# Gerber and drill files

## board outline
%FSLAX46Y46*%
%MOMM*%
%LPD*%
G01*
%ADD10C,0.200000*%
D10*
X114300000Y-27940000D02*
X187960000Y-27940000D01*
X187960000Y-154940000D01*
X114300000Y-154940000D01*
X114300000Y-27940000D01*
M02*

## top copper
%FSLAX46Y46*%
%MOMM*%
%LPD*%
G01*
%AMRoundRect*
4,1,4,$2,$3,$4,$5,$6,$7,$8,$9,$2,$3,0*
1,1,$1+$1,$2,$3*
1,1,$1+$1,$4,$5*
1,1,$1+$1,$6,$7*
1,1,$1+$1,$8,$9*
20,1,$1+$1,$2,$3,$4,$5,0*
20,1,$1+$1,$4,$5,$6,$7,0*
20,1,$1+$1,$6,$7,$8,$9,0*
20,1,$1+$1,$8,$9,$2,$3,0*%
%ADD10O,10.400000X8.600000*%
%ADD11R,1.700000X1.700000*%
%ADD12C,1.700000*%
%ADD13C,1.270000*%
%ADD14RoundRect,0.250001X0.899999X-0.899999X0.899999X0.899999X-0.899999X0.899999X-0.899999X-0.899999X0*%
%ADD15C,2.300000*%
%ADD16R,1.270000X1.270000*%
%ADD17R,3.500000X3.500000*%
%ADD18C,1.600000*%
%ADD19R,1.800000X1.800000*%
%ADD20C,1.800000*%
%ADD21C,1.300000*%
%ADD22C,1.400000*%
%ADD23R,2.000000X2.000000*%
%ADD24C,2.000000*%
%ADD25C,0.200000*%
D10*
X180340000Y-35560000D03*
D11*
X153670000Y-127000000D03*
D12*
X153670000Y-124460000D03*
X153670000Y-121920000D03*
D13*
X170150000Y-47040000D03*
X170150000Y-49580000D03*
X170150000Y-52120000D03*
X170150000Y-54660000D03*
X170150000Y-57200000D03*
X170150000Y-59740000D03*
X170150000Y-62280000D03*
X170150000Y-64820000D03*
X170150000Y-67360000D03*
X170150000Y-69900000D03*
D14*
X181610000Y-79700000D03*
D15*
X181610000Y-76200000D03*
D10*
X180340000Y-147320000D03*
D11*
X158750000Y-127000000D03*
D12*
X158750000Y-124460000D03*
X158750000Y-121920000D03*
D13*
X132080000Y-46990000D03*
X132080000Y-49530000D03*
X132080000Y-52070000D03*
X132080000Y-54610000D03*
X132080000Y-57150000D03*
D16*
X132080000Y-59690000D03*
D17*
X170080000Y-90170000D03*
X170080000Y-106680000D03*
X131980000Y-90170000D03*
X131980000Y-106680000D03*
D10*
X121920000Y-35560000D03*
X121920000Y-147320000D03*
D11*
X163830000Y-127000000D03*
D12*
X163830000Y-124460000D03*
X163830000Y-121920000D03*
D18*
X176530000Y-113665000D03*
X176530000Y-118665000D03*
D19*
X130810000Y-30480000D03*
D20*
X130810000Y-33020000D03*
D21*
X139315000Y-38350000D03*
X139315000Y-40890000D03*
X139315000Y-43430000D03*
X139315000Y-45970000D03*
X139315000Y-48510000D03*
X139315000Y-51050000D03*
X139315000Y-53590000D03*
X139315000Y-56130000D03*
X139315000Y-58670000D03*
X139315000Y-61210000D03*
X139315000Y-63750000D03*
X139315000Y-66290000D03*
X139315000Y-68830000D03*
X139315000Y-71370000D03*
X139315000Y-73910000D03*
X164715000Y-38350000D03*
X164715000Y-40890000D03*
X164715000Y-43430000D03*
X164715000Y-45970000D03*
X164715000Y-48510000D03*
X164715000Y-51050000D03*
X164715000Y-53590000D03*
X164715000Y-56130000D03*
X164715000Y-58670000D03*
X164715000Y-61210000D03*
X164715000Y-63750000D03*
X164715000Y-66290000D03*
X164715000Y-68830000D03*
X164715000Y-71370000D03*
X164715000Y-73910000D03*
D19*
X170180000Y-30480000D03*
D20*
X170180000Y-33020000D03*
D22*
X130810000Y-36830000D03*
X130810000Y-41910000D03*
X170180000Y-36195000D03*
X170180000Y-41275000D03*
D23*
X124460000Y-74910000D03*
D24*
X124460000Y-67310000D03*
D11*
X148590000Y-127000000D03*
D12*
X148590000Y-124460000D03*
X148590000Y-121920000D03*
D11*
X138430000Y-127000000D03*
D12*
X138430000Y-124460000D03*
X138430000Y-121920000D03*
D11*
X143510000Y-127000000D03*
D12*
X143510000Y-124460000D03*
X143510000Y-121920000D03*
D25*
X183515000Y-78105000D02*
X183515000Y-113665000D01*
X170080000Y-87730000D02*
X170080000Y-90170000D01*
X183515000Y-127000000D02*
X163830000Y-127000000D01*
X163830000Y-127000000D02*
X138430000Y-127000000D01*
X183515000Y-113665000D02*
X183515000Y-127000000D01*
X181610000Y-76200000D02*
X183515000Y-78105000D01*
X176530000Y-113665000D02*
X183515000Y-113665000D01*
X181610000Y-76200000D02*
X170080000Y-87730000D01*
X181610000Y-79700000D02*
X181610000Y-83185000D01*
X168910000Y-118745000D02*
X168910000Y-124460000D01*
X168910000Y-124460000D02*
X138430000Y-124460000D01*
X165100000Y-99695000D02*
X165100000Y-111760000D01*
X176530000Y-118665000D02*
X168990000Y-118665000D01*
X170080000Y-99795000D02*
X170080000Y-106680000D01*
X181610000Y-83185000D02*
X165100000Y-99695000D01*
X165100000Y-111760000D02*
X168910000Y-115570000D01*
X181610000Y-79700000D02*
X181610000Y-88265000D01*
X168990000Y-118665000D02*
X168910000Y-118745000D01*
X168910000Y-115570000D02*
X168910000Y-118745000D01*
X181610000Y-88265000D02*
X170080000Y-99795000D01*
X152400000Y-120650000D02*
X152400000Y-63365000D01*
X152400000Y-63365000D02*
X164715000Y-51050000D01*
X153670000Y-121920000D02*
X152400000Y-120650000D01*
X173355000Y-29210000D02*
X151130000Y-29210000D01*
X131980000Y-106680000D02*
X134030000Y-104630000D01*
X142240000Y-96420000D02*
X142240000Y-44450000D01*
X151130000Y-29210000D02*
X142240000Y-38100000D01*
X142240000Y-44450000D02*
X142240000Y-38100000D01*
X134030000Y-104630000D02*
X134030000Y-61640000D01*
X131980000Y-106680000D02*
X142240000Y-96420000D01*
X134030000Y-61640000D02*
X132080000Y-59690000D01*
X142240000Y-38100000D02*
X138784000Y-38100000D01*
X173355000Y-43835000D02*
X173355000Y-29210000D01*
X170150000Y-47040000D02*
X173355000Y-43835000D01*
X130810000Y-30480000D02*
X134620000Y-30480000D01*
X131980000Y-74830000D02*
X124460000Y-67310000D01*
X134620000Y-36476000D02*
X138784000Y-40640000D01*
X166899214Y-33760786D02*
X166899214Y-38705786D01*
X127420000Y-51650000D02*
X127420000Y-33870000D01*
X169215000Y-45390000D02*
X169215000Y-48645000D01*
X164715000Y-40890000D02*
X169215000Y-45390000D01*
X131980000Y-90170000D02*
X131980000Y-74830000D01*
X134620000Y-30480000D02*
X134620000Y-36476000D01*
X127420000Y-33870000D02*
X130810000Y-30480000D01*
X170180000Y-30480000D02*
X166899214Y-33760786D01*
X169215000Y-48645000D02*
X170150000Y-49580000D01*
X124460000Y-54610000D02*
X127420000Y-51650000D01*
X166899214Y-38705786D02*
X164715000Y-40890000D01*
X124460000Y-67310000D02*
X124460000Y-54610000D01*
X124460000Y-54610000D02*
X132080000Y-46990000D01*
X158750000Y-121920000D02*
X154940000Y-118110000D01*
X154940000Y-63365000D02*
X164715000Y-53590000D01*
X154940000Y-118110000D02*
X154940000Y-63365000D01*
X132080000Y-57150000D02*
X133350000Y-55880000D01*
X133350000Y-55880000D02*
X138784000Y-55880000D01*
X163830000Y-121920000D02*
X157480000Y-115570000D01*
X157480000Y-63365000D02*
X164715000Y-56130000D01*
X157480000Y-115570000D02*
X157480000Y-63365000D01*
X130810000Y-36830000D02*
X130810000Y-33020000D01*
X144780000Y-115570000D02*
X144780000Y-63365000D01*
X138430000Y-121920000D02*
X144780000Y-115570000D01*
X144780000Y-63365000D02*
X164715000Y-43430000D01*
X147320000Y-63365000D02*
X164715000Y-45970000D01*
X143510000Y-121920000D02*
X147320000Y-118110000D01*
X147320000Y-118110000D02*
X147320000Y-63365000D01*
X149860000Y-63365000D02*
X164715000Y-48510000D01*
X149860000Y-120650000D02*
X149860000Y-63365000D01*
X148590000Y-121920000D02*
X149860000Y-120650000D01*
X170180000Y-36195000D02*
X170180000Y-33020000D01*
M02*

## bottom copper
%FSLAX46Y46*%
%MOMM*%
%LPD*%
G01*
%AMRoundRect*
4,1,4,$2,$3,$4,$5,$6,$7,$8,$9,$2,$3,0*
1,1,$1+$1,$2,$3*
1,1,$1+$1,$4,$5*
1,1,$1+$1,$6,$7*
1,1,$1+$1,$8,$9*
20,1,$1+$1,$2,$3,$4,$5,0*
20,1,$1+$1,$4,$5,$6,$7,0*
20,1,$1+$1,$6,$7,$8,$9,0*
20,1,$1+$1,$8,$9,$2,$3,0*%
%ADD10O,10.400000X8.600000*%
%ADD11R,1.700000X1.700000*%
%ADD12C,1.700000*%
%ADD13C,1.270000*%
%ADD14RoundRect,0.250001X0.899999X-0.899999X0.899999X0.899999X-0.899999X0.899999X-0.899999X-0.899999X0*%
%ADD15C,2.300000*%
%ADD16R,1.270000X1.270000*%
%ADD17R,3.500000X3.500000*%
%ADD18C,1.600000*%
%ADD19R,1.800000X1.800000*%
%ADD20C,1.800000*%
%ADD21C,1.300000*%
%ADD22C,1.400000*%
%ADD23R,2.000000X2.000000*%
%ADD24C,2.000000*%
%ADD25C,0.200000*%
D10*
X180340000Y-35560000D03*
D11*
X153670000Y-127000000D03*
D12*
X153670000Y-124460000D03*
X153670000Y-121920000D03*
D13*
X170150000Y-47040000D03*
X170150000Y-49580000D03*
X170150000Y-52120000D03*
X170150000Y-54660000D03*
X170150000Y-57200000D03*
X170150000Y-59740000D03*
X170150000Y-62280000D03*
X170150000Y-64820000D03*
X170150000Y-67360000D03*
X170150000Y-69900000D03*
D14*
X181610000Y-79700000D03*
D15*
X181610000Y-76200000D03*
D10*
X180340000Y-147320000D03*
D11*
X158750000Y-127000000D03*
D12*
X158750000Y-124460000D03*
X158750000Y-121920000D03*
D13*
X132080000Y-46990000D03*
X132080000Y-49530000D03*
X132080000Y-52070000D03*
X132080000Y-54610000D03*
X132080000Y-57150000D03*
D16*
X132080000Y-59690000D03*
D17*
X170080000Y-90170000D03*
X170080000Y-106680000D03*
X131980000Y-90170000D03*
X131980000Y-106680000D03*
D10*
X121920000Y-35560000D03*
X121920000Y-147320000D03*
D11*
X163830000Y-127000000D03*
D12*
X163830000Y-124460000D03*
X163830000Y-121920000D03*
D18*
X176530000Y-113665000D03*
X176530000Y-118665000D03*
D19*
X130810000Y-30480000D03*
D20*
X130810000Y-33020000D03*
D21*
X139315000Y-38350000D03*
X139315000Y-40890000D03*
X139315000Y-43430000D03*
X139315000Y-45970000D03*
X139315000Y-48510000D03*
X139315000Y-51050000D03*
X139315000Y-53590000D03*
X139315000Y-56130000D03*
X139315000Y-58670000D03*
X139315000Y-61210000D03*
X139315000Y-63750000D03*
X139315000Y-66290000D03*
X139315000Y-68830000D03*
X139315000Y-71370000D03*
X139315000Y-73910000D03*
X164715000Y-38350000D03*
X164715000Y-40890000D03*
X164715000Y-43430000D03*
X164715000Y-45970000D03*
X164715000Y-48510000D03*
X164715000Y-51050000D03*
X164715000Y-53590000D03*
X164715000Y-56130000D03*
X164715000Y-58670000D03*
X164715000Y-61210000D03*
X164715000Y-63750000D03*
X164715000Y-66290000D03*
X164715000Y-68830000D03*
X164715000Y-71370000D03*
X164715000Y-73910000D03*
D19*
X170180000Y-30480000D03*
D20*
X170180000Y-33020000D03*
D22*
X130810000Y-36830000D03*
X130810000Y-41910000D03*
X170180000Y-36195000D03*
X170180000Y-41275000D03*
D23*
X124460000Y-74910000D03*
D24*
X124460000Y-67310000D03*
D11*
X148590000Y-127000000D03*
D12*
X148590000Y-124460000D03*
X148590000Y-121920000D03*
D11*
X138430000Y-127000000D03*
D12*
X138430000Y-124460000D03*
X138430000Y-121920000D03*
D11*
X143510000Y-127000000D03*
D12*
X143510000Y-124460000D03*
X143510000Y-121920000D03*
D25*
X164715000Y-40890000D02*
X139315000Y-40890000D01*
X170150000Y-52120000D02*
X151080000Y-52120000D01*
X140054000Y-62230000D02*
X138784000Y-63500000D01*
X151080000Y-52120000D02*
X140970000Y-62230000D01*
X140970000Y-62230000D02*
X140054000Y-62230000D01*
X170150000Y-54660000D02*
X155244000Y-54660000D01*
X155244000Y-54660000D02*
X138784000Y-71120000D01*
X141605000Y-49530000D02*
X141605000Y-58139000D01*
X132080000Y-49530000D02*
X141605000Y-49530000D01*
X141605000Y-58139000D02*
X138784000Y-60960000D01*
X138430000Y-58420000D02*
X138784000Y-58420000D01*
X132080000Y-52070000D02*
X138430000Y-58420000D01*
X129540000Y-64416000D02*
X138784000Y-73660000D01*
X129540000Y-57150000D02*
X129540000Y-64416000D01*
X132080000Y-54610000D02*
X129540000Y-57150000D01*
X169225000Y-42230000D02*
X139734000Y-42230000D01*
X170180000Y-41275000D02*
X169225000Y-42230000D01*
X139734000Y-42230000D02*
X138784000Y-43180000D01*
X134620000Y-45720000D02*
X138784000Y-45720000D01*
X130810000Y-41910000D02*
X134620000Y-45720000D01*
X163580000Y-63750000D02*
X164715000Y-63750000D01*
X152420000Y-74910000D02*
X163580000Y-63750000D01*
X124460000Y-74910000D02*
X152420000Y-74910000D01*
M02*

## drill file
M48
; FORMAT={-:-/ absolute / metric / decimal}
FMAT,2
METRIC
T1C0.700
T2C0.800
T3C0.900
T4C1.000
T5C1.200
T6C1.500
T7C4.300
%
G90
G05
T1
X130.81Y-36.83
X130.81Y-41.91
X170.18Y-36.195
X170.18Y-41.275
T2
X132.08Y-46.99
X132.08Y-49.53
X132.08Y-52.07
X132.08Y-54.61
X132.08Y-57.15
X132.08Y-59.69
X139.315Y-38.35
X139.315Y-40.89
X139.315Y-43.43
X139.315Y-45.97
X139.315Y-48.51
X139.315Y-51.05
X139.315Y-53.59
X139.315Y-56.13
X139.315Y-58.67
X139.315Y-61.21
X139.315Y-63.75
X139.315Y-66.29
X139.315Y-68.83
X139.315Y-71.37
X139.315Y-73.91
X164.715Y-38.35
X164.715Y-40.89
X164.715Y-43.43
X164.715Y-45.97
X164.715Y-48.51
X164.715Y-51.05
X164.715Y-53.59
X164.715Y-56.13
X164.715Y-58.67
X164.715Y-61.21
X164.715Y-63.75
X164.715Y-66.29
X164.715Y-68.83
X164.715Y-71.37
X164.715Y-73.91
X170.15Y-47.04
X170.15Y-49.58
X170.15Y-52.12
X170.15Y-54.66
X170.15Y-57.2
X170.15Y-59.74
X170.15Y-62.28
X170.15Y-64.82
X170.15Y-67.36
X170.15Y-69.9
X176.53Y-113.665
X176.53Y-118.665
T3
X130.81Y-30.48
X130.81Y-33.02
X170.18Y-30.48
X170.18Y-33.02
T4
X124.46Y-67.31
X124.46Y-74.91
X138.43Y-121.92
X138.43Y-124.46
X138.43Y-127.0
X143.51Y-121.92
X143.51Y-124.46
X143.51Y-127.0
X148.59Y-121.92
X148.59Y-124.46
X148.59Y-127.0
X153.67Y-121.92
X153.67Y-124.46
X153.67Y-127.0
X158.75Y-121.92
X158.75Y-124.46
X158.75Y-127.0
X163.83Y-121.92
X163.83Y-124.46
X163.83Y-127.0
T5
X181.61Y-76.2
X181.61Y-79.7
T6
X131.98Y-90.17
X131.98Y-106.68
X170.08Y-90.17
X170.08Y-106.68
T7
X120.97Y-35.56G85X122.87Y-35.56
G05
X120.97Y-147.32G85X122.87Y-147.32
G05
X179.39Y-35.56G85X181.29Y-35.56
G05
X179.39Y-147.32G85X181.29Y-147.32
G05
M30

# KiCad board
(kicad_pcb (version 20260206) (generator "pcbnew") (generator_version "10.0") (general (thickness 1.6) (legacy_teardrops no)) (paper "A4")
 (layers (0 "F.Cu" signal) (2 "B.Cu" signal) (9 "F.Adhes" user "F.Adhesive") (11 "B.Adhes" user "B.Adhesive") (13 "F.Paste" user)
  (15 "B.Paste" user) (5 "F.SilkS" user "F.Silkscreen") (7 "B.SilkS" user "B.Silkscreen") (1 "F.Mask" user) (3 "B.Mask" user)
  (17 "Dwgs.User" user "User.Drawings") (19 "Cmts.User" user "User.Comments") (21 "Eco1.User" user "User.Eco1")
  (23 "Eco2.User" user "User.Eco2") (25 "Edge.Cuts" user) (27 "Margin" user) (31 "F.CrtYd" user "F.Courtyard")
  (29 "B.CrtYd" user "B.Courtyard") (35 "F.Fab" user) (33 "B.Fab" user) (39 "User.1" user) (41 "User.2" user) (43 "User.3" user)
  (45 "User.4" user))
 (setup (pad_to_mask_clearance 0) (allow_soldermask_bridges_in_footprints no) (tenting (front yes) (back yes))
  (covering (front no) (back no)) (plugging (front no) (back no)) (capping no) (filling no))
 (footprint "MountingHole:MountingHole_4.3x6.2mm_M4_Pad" (layer "F.Cu") (at 180.34 35.56)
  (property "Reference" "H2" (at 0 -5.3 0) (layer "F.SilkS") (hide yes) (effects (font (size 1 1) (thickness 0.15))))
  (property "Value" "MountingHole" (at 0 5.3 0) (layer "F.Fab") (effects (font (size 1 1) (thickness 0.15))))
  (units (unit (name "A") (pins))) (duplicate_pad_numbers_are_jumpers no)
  (pad "1" thru_hole oval (at 0 0) (size 10.4 8.6) (drill oval 6.2 4.3) (layers "*.Cu" "*.Mask") (remove_unused_layers no)))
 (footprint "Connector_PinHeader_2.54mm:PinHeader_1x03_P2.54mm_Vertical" (layer "F.Cu") (at 153.67 127 180)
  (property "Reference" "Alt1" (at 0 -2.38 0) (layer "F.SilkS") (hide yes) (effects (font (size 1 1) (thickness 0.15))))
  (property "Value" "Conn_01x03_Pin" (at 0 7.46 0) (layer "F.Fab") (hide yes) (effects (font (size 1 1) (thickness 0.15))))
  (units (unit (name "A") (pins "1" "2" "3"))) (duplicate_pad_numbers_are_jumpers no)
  (pad "1" thru_hole rect (at 0 0 180) (size 1.7 1.7) (drill 1) (layers "*.Cu" "*.Mask") (remove_unused_layers no) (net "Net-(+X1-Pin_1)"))
  (pad "2" thru_hole circle (at 0 2.54 180) (size 1.7 1.7) (drill 1) (layers "*.Cu" "*.Mask") (remove_unused_layers no)
   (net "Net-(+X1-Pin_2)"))
  (pad "3" thru_hole circle (at 0 5.08 180) (size 1.7 1.7) (drill 1) (layers "*.Cu" "*.Mask") (remove_unused_layers no)
   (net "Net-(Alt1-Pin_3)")))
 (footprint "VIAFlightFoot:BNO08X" (layer "F.Cu") (at 168.88 45.77)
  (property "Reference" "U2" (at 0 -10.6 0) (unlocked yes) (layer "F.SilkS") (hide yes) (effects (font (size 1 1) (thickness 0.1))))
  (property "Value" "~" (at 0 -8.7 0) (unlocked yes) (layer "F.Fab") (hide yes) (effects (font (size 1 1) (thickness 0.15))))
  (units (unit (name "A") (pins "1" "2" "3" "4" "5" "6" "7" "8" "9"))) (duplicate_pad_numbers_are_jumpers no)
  (pad "1" thru_hole circle (at 1.27 1.27) (size 1.27 1.27) (drill 0.8) (layers "*.Cu" "*.Mask") (remove_unused_layers no) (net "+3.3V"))
  (pad "2" thru_hole circle (at 1.27 3.81) (size 1.27 1.27) (drill 0.8) (layers "*.Cu" "*.Mask") (remove_unused_layers no) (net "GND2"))
  (pad "3" thru_hole circle (at 1.27 6.35) (size 1.27 1.27) (drill 0.8) (layers "*.Cu" "*.Mask") (remove_unused_layers no)
   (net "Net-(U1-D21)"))
  (pad "4" thru_hole circle (at 1.27 8.89) (size 1.27 1.27) (drill 0.8) (layers "*.Cu" "*.Mask") (remove_unused_layers no)
   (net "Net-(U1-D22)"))
  (pad "5" thru_hole circle (at 1.27 11.43) (size 1.27 1.27) (drill 0.8) (layers "*.Cu" "*.Mask") (remove_unused_layers no)
   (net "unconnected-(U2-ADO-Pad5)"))
  (pad "6" thru_hole circle (at 1.27 13.97) (size 1.27 1.27) (drill 0.8) (layers "*.Cu" "*.Mask") (remove_unused_layers no)
   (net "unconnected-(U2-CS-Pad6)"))
  (pad "7" thru_hole circle (at 1.27 16.51) (size 1.27 1.27) (drill 0.8) (layers "*.Cu" "*.Mask") (remove_unused_layers no)
   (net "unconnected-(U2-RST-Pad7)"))
  (pad "8" thru_hole circle (at 1.27 19.05) (size 1.27 1.27) (drill 0.8) (layers "*.Cu" "*.Mask") (remove_unused_layers no)
   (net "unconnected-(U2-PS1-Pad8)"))
  (pad "9" thru_hole circle (at 1.27 21.59) (size 1.27 1.27) (drill 0.8) (layers "*.Cu" "*.Mask") (remove_unused_layers no)
   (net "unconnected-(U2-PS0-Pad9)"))
  (pad "10" thru_hole circle (at 1.27 24.13) (size 1.27 1.27) (drill 0.8) (layers "*.Cu" "*.Mask") (remove_unused_layers no)))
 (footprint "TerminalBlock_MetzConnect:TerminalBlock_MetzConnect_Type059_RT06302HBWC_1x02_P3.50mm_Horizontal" (layer "F.Cu")
  (at 181.61 79.7 90)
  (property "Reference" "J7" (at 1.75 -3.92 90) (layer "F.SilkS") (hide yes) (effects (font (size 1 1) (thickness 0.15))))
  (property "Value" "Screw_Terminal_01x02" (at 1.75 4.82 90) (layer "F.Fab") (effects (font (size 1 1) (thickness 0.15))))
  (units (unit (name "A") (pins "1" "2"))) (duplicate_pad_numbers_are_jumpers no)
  (pad "1" thru_hole roundrect (at 0 0 90) (size 2.3 2.3) (drill 1.2) (layers "*.Cu" "*.Mask") (remove_unused_layers no)
   (roundrect_rratio 0.108696) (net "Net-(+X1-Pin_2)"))
  (pad "2" thru_hole circle (at 3.5 0 90) (size 2.3 2.3) (drill 1.2) (layers "*.Cu" "*.Mask") (remove_unused_layers no)
   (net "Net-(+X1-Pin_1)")))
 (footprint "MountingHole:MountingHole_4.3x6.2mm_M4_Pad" (layer "F.Cu") (at 180.34 147.32)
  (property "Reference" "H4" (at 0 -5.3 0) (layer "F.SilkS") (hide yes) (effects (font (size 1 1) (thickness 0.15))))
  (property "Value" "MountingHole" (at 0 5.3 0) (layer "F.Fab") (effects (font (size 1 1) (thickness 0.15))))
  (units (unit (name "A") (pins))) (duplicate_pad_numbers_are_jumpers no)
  (pad "1" thru_hole oval (at 0 0) (size 10.4 8.6) (drill oval 6.2 4.3) (layers "*.Cu" "*.Mask") (remove_unused_layers no)))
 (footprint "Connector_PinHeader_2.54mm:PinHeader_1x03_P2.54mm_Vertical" (layer "F.Cu") (at 158.75 127 180)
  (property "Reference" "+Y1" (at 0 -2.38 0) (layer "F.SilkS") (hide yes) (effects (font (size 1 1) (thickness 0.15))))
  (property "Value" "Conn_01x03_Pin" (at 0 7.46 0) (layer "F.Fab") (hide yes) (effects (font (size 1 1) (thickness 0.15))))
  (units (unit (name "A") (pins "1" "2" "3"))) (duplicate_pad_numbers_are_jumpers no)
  (pad "1" thru_hole rect (at 0 0 180) (size 1.7 1.7) (drill 1) (layers "*.Cu" "*.Mask") (remove_unused_layers no) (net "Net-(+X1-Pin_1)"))
  (pad "2" thru_hole circle (at 0 2.54 180) (size 1.7 1.7) (drill 1) (layers "*.Cu" "*.Mask") (remove_unused_layers no)
   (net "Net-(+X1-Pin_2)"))
  (pad "3" thru_hole circle (at 0 5.08 180) (size 1.7 1.7) (drill 1) (layers "*.Cu" "*.Mask") (remove_unused_layers no)
   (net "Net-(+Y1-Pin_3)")))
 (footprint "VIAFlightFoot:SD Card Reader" (layer "F.Cu") (at 133.35 45.72 -90)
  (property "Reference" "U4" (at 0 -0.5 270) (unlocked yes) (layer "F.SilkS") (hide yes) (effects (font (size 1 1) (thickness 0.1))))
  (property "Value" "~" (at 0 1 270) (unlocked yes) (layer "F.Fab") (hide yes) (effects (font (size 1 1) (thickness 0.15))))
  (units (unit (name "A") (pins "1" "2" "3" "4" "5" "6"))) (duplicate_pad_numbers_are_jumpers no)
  (pad "1" thru_hole circle (at 1.27 1.27 270) (size 1.27 1.27) (drill 0.8) (layers "*.Cu" "*.Mask") (remove_unused_layers no) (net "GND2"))
  (pad "2" thru_hole circle (at 3.81 1.27 270) (size 1.27 1.27) (drill 0.8) (layers "*.Cu" "*.Mask") (remove_unused_layers no)
   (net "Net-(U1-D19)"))
  (pad "3" thru_hole circle (at 6.35 1.27 270) (size 1.27 1.27) (drill 0.8) (layers "*.Cu" "*.Mask") (remove_unused_layers no)
   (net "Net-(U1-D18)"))
  (pad "4" thru_hole circle (at 8.89 1.27 270) (size 1.27 1.27) (drill 0.8) (layers "*.Cu" "*.Mask") (remove_unused_layers no)
   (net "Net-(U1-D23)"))
  (pad "5" thru_hole circle (at 11.43 1.27 270) (size 1.27 1.27) (drill 0.8) (layers "*.Cu" "*.Mask") (remove_unused_layers no)
   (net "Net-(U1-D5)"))
  (pad "6" thru_hole rect (at 13.97 1.27 270) (size 1.27 1.27) (drill 0.8) (layers "*.Cu" "*.Mask") (remove_unused_layers no) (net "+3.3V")))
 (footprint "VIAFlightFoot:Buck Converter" (layer "F.Cu") (at 172.62 87.63 -90)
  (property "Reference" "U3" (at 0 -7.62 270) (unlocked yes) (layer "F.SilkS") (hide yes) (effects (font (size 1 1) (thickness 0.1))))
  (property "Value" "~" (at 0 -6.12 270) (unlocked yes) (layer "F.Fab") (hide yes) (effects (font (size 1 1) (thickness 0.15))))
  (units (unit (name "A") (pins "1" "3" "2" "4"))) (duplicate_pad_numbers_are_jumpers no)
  (pad "1" thru_hole rect (at 2.54 2.54 270) (size 3.5 3.5) (drill 1.5) (layers "*.Cu" "*.Mask") (remove_unused_layers no)
   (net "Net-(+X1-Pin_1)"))
  (pad "2" thru_hole rect (at 19.05 2.54 270) (size 3.5 3.5) (drill 1.5) (layers "*.Cu" "*.Mask") (remove_unused_layers no)
   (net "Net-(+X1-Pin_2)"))
  (pad "3" thru_hole rect (at 2.54 40.64 270) (size 3.5 3.5) (drill 1.5) (layers "*.Cu" "*.Mask") (remove_unused_layers no) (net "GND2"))
  (pad "4" thru_hole rect (at 19.05 40.64 270) (size 3.5 3.5) (drill 1.5) (layers "*.Cu" "*.Mask") (remove_unused_layers no) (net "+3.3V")))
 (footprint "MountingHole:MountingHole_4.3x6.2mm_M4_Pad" (layer "F.Cu") (at 121.92 35.56)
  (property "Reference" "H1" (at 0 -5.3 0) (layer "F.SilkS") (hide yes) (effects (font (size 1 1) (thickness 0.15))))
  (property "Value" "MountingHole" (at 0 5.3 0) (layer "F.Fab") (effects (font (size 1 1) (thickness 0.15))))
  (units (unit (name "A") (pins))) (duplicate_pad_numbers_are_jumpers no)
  (pad "1" thru_hole oval (at 0 0) (size 10.4 8.6) (drill oval 6.2 4.3) (layers "*.Cu" "*.Mask") (remove_unused_layers no)))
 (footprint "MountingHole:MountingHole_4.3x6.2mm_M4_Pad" (layer "F.Cu") (at 121.92 147.32)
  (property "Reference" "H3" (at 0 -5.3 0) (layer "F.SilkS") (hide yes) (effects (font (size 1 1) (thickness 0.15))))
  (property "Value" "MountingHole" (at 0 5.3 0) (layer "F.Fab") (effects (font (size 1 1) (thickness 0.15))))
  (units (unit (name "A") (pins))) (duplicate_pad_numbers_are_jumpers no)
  (pad "1" thru_hole oval (at 0 0) (size 10.4 8.6) (drill oval 6.2 4.3) (layers "*.Cu" "*.Mask") (remove_unused_layers no)))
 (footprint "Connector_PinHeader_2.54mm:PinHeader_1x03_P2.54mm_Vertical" (layer "F.Cu") (at 163.83 127 180)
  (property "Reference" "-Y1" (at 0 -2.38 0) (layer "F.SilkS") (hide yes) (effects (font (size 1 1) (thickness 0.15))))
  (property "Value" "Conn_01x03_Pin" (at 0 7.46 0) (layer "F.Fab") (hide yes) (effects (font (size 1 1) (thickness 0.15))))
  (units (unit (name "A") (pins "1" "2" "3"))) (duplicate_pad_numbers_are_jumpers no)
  (pad "1" thru_hole rect (at 0 0 180) (size 1.7 1.7) (drill 1) (layers "*.Cu" "*.Mask") (remove_unused_layers no) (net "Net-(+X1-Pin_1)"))
  (pad "2" thru_hole circle (at 0 2.54 180) (size 1.7 1.7) (drill 1) (layers "*.Cu" "*.Mask") (remove_unused_layers no)
   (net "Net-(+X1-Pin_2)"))
  (pad "3" thru_hole circle (at 0 5.08 180) (size 1.7 1.7) (drill 1) (layers "*.Cu" "*.Mask") (remove_unused_layers no)
   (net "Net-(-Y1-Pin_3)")))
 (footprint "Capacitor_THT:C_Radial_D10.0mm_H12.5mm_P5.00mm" (layer "F.Cu") (at 176.53 113.665 -90)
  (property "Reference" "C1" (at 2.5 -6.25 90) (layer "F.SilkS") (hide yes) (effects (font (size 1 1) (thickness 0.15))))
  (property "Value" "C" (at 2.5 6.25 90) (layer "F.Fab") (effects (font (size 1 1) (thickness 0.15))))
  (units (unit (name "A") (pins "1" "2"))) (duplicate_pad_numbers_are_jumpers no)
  (pad "1" thru_hole circle (at 0 0 270) (size 1.6 1.6) (drill 0.8) (layers "*.Cu" "*.Mask") (remove_unused_layers no)
   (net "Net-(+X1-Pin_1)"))
  (pad "2" thru_hole circle (at 5 0 270) (size 1.6 1.6) (drill 0.8) (layers "*.Cu" "*.Mask") (remove_unused_layers no)
   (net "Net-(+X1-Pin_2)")))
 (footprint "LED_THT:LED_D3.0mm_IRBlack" (layer "F.Cu") (at 130.81 30.48 -90)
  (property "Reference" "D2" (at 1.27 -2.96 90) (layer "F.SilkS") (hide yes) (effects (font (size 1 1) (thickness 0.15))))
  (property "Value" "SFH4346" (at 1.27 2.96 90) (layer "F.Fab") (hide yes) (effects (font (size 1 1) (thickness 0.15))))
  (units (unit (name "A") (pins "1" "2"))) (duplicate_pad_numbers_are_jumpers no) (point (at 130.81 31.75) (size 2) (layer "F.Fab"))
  (pad "1" thru_hole rect (at 0 0 270) (size 1.8 1.8) (drill 0.9) (layers "*.Cu" "*.Mask") (remove_unused_layers no) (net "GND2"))
  (pad "2" thru_hole circle (at 2.54 0 270) (size 1.8 1.8) (drill 0.9) (layers "*.Cu" "*.Mask") (remove_unused_layers no) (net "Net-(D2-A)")))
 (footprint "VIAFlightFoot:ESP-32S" (layer "F.Cu") (at 136.775 28.19)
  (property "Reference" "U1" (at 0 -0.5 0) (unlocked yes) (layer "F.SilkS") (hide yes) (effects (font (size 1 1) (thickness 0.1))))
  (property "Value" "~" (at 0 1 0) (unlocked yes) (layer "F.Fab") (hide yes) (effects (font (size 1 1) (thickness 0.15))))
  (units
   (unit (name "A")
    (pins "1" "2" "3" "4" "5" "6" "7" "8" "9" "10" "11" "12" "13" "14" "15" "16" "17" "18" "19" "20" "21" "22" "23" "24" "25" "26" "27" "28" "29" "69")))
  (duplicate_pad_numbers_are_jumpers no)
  (pad "1" thru_hole circle (at 2.54 10.16) (size 1.3 1.3) (drill 0.8) (layers "*.Cu" "*.Mask") (remove_unused_layers no) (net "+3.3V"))
  (pad "2" thru_hole circle (at 2.54 12.7) (size 1.3 1.3) (drill 0.8) (layers "*.Cu" "*.Mask") (remove_unused_layers no) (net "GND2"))
  (pad "3" thru_hole circle (at 2.54 15.24) (size 1.3 1.3) (drill 0.8) (layers "*.Cu" "*.Mask") (remove_unused_layers no)
   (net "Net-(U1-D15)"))
  (pad "4" thru_hole circle (at 2.54 17.78) (size 1.3 1.3) (drill 0.8) (layers "*.Cu" "*.Mask") (remove_unused_layers no)
   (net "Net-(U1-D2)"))
  (pad "5" thru_hole circle (at 2.54 20.32) (size 1.3 1.3) (drill 0.8) (layers "*.Cu" "*.Mask") (remove_unused_layers no)
   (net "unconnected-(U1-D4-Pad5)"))
  (pad "6" thru_hole circle (at 2.54 22.86) (size 1.3 1.3) (drill 0.8) (layers "*.Cu" "*.Mask") (remove_unused_layers no)
   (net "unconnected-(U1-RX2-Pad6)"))
  (pad "7" thru_hole circle (at 2.54 25.4) (size 1.3 1.3) (drill 0.8) (layers "*.Cu" "*.Mask") (remove_unused_layers no)
   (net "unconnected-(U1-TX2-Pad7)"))
  (pad "8" thru_hole circle (at 2.54 27.94) (size 1.3 1.3) (drill 0.8) (layers "*.Cu" "*.Mask") (remove_unused_layers no)
   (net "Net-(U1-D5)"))
  (pad "9" thru_hole circle (at 2.54 30.48) (size 1.3 1.3) (drill 0.8) (layers "*.Cu" "*.Mask") (remove_unused_layers no)
   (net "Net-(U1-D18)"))
  (pad "10" thru_hole circle (at 2.54 33.02) (size 1.3 1.3) (drill 0.8) (layers "*.Cu" "*.Mask") (remove_unused_layers no)
   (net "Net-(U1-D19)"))
  (pad "11" thru_hole circle (at 2.54 35.56) (size 1.3 1.3) (drill 0.8) (layers "*.Cu" "*.Mask") (remove_unused_layers no)
   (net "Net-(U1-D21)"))
  (pad "12" thru_hole circle (at 2.54 38.1) (size 1.3 1.3) (drill 0.8) (layers "*.Cu" "*.Mask") (remove_unused_layers no)
   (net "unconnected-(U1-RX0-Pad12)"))
  (pad "13" thru_hole circle (at 2.54 40.64) (size 1.3 1.3) (drill 0.8) (layers "*.Cu" "*.Mask") (remove_unused_layers no)
   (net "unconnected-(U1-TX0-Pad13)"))
  (pad "14" thru_hole circle (at 2.54 43.18) (size 1.3 1.3) (drill 0.8) (layers "*.Cu" "*.Mask") (remove_unused_layers no)
   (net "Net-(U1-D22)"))
  (pad "15" thru_hole circle (at 2.54 45.72) (size 1.3 1.3) (drill 0.8) (layers "*.Cu" "*.Mask") (remove_unused_layers no)
   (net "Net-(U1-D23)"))
  (pad "16" thru_hole circle (at 27.94 10.16) (size 1.3 1.3) (drill 0.8) (layers "*.Cu" "*.Mask") (remove_unused_layers no)
   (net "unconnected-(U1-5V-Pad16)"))
  (pad "17" thru_hole circle (at 27.94 12.7) (size 1.3 1.3) (drill 0.8) (layers "*.Cu" "*.Mask") (remove_unused_layers no) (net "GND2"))
  (pad "18" thru_hole circle (at 27.94 15.24) (size 1.3 1.3) (drill 0.8) (layers "*.Cu" "*.Mask") (remove_unused_layers no)
   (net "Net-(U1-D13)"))
  (pad "19" thru_hole circle (at 27.94 17.78) (size 1.3 1.3) (drill 0.8) (layers "*.Cu" "*.Mask") (remove_unused_layers no)
   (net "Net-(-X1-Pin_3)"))
  (pad "20" thru_hole circle (at 27.94 20.32) (size 1.3 1.3) (drill 0.8) (layers "*.Cu" "*.Mask") (remove_unused_layers no)
   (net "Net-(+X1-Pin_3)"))
  (pad "21" thru_hole circle (at 27.94 22.86) (size 1.3 1.3) (drill 0.8) (layers "*.Cu" "*.Mask") (remove_unused_layers no)
   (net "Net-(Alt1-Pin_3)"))
  (pad "22" thru_hole circle (at 27.94 25.4) (size 1.3 1.3) (drill 0.8) (layers "*.Cu" "*.Mask") (remove_unused_layers no)
   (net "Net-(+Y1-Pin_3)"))
  (pad "23" thru_hole circle (at 27.94 27.94) (size 1.3 1.3) (drill 0.8) (layers "*.Cu" "*.Mask") (remove_unused_layers no)
   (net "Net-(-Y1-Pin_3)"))
  (pad "24" thru_hole circle (at 27.94 30.48) (size 1.3 1.3) (drill 0.8) (layers "*.Cu" "*.Mask") (remove_unused_layers no)
   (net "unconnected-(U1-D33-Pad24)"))
  (pad "25" thru_hole circle (at 27.94 33.02) (size 1.3 1.3) (drill 0.8) (layers "*.Cu" "*.Mask") (remove_unused_layers no)
   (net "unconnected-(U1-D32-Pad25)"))
  (pad "26" thru_hole circle (at 27.94 35.56) (size 1.3 1.3) (drill 0.8) (layers "*.Cu" "*.Mask") (remove_unused_layers no)
   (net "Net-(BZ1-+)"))
  (pad "27" thru_hole circle (at 27.94 38.1) (size 1.3 1.3) (drill 0.8) (layers "*.Cu" "*.Mask") (remove_unused_layers no)
   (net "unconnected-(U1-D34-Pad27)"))
  (pad "28" thru_hole circle (at 27.94 40.64) (size 1.3 1.3) (drill 0.8) (layers "*.Cu" "*.Mask") (remove_unused_layers no)
   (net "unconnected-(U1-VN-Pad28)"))
  (pad "29" thru_hole circle (at 27.94 43.18) (size 1.3 1.3) (drill 0.8) (layers "*.Cu" "*.Mask") (remove_unused_layers no)
   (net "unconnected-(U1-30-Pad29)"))
  (pad "30" thru_hole circle (at 27.94 45.72) (size 1.3 1.3) (drill 0.8) (layers "*.Cu" "*.Mask") (remove_unused_layers no)))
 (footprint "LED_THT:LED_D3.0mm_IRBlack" (layer "F.Cu") (at 170.18 30.48 -90)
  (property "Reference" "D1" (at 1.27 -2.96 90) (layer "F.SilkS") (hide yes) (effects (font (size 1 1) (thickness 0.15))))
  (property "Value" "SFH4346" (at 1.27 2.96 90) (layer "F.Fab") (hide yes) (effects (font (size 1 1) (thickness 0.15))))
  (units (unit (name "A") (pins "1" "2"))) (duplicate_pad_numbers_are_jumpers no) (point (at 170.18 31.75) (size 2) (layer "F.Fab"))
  (pad "1" thru_hole rect (at 0 0 270) (size 1.8 1.8) (drill 0.9) (layers "*.Cu" "*.Mask") (remove_unused_layers no) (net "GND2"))
  (pad "2" thru_hole circle (at 2.54 0 270) (size 1.8 1.8) (drill 0.9) (layers "*.Cu" "*.Mask") (remove_unused_layers no) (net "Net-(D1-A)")))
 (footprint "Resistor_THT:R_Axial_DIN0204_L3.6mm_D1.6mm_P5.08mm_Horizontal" (layer "F.Cu") (at 130.81 36.83 -90)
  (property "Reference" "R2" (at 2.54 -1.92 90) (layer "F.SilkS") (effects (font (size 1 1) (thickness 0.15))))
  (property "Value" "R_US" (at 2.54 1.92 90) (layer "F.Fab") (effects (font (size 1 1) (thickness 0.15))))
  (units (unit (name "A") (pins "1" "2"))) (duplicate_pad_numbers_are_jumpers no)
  (pad "1" thru_hole circle (at 0 0 270) (size 1.4 1.4) (drill 0.7) (layers "*.Cu" "*.Mask") (remove_unused_layers no) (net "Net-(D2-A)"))
  (pad "2" thru_hole circle (at 5.08 0 270) (size 1.4 1.4) (drill 0.7) (layers "*.Cu" "*.Mask") (remove_unused_layers no)
   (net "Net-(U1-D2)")))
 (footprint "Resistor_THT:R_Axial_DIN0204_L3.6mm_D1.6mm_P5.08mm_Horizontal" (layer "F.Cu") (at 170.18 36.195 -90)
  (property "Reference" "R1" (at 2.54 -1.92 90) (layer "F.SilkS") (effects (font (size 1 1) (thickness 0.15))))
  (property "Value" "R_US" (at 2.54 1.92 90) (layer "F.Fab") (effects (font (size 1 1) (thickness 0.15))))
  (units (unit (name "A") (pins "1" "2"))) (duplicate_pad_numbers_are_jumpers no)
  (pad "1" thru_hole circle (at 0 0 270) (size 1.4 1.4) (drill 0.7) (layers "*.Cu" "*.Mask") (remove_unused_layers no) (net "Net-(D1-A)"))
  (pad "2" thru_hole circle (at 5.08 0 270) (size 1.4 1.4) (drill 0.7) (layers "*.Cu" "*.Mask") (remove_unused_layers no)
   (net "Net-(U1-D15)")))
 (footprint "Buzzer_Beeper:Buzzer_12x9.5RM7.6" (layer "F.Cu") (at 124.46 74.91 90)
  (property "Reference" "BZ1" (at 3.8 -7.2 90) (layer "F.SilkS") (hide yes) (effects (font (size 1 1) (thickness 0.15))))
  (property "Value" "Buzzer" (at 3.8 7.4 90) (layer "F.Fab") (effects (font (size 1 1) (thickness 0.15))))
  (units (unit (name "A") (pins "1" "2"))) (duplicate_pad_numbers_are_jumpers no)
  (pad "1" thru_hole rect (at 0 0 90) (size 2 2) (drill 1) (layers "*.Cu" "*.Mask") (remove_unused_layers no) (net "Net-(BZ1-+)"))
  (pad "2" thru_hole circle (at 7.6 0 90) (size 2 2) (drill 1) (layers "*.Cu" "*.Mask") (remove_unused_layers no) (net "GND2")))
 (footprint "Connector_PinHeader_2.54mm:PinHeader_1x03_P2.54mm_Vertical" (layer "F.Cu") (at 148.59 127 180)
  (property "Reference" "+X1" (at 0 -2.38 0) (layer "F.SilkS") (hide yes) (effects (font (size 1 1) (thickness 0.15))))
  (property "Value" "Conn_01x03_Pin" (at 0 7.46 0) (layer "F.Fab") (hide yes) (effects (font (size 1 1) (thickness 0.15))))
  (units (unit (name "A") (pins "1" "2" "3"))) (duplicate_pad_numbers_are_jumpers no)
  (pad "1" thru_hole rect (at 0 0 180) (size 1.7 1.7) (drill 1) (layers "*.Cu" "*.Mask") (remove_unused_layers no) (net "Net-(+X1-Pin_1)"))
  (pad "2" thru_hole circle (at 0 2.54 180) (size 1.7 1.7) (drill 1) (layers "*.Cu" "*.Mask") (remove_unused_layers no)
   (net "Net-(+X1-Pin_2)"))
  (pad "3" thru_hole circle (at 0 5.08 180) (size 1.7 1.7) (drill 1) (layers "*.Cu" "*.Mask") (remove_unused_layers no)
   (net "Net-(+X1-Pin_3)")))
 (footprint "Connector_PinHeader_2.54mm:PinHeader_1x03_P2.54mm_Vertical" (layer "F.Cu") (at 138.43 127 180)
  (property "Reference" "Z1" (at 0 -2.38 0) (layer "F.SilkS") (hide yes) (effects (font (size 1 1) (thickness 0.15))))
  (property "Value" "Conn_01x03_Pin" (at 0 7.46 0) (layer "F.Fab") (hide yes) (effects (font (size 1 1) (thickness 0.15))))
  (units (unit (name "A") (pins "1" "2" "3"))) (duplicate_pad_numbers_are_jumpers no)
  (pad "1" thru_hole rect (at 0 0 180) (size 1.7 1.7) (drill 1) (layers "*.Cu" "*.Mask") (remove_unused_layers no) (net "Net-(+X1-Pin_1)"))
  (pad "2" thru_hole circle (at 0 2.54 180) (size 1.7 1.7) (drill 1) (layers "*.Cu" "*.Mask") (remove_unused_layers no)
   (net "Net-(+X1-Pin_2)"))
  (pad "3" thru_hole circle (at 0 5.08 180) (size 1.7 1.7) (drill 1) (layers "*.Cu" "*.Mask") (remove_unused_layers no) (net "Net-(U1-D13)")))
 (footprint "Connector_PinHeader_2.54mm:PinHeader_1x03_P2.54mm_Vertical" (layer "F.Cu") (at 143.51 127 180)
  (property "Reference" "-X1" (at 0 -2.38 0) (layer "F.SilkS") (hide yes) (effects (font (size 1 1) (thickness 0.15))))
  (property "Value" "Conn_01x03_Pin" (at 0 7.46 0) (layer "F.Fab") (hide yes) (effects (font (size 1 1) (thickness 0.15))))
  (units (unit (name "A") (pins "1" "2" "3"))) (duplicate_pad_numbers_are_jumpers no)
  (pad "1" thru_hole rect (at 0 0 180) (size 1.7 1.7) (drill 1) (layers "*.Cu" "*.Mask") (remove_unused_layers no) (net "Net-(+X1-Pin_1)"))
  (pad "2" thru_hole circle (at 0 2.54 180) (size 1.7 1.7) (drill 1) (layers "*.Cu" "*.Mask") (remove_unused_layers no)
   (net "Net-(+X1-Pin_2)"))
  (pad "3" thru_hole circle (at 0 5.08 180) (size 1.7 1.7) (drill 1) (layers "*.Cu" "*.Mask") (remove_unused_layers no)
   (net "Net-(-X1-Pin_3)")))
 (gr_rect (start 114.3 27.94) (end 187.96 154.94) (stroke (width 0.2) (type solid)) (fill no) (layer "Edge.Cuts"))
 (segment (start 183.515 78.105) (end 183.515 113.665) (width 0.2) (layer "F.Cu") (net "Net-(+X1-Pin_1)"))
 (segment (start 170.08 87.73) (end 170.08 90.17) (width 0.2) (layer "F.Cu") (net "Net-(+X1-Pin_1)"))
 (segment (start 183.515 127) (end 163.83 127) (width 0.2) (layer "F.Cu") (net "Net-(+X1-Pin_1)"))
 (segment (start 163.83 127) (end 138.43 127) (width 0.2) (layer "F.Cu") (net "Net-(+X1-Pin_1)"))
 (segment (start 183.515 113.665) (end 183.515 127) (width 0.2) (layer "F.Cu") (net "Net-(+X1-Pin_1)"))
 (segment (start 181.61 76.2) (end 183.515 78.105) (width 0.2) (layer "F.Cu") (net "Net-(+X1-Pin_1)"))
 (segment (start 176.53 113.665) (end 183.515 113.665) (width 0.2) (layer "F.Cu") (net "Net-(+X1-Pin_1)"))
 (segment (start 181.61 76.2) (end 170.08 87.73) (width 0.2) (layer "F.Cu") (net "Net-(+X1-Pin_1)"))
 (segment (start 181.61 79.7) (end 181.61 83.185) (width 0.2) (layer "F.Cu") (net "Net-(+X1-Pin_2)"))
 (segment (start 168.91 118.745) (end 168.91 124.46) (width 0.2) (layer "F.Cu") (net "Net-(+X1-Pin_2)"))
 (segment (start 168.91 124.46) (end 138.43 124.46) (width 0.2) (layer "F.Cu") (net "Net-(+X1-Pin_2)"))
 (segment (start 165.1 99.695) (end 165.1 111.76) (width 0.2) (layer "F.Cu") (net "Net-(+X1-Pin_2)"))
 (segment (start 176.53 118.665) (end 168.99 118.665) (width 0.2) (layer "F.Cu") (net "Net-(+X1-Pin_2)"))
 (segment (start 170.08 99.795) (end 170.08 106.68) (width 0.2) (layer "F.Cu") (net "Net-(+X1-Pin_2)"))
 (segment (start 181.61 83.185) (end 165.1 99.695) (width 0.2) (layer "F.Cu") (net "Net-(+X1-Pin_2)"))
 (segment (start 165.1 111.76) (end 168.91 115.57) (width 0.2) (layer "F.Cu") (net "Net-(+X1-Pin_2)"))
 (segment (start 181.61 79.7) (end 181.61 88.265) (width 0.2) (layer "F.Cu") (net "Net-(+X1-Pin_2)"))
 (segment (start 168.99 118.665) (end 168.91 118.745) (width 0.2) (layer "F.Cu") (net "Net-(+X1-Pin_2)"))
 (segment (start 168.91 115.57) (end 168.91 118.745) (width 0.2) (layer "F.Cu") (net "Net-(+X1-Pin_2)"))
 (segment (start 181.61 88.265) (end 170.08 99.795) (width 0.2) (layer "F.Cu") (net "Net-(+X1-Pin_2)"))
 (segment (start 152.4 120.65) (end 152.4 63.365) (width 0.2) (layer "F.Cu") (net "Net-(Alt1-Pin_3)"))
 (segment (start 152.4 63.365) (end 164.715 51.05) (width 0.2) (layer "F.Cu") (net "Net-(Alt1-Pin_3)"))
 (segment (start 153.67 121.92) (end 152.4 120.65) (width 0.2) (layer "F.Cu") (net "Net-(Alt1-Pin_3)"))
 (segment (start 173.355 29.21) (end 151.13 29.21) (width 0.2) (layer "F.Cu") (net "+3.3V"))
 (segment (start 131.98 106.68) (end 134.03 104.63) (width 0.2) (layer "F.Cu") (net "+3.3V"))
 (segment (start 142.24 96.42) (end 142.24 44.45) (width 0.2) (layer "F.Cu") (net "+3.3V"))
 (segment (start 151.13 29.21) (end 142.24 38.1) (width 0.2) (layer "F.Cu") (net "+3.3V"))
 (segment (start 142.24 44.45) (end 142.24 38.1) (width 0.2) (layer "F.Cu") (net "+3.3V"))
 (segment (start 134.03 104.63) (end 134.03 61.64) (width 0.2) (layer "F.Cu") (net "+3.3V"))
 (segment (start 131.98 106.68) (end 142.24 96.42) (width 0.2) (layer "F.Cu") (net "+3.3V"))
 (segment (start 134.03 61.64) (end 132.08 59.69) (width 0.2) (layer "F.Cu") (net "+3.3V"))
 (segment (start 142.24 38.1) (end 138.784 38.1) (width 0.2) (layer "F.Cu") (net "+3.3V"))
 (segment (start 173.355 43.835) (end 173.355 29.21) (width 0.2) (layer "F.Cu") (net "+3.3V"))
 (segment (start 170.15 47.04) (end 173.355 43.835) (width 0.2) (layer "F.Cu") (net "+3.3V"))
 (segment (start 130.81 30.48) (end 134.62 30.48) (width 0.2) (layer "F.Cu") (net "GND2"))
 (segment (start 131.98 74.83) (end 124.46 67.31) (width 0.2) (layer "F.Cu") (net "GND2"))
 (segment (start 134.62 36.476) (end 138.784 40.64) (width 0.2) (layer "F.Cu") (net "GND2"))
 (segment (start 166.899214 33.760786) (end 166.899214 38.705786) (width 0.2) (layer "F.Cu") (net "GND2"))
 (segment (start 127.42 51.65) (end 127.42 33.87) (width 0.2) (layer "F.Cu") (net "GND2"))
 (segment (start 169.215 45.39) (end 169.215 48.645) (width 0.2) (layer "F.Cu") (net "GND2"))
 (segment (start 164.715 40.89) (end 169.215 45.39) (width 0.2) (layer "F.Cu") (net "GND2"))
 (segment (start 131.98 90.17) (end 131.98 74.83) (width 0.2) (layer "F.Cu") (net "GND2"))
 (segment (start 134.62 30.48) (end 134.62 36.476) (width 0.2) (layer "F.Cu") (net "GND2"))
 (segment (start 127.42 33.87) (end 130.81 30.48) (width 0.2) (layer "F.Cu") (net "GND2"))
 (segment (start 170.18 30.48) (end 166.899214 33.760786) (width 0.2) (layer "F.Cu") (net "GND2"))
 (segment (start 169.215 48.645) (end 170.15 49.58) (width 0.2) (layer "F.Cu") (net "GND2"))
 (segment (start 124.46 54.61) (end 127.42 51.65) (width 0.2) (layer "F.Cu") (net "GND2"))
 (segment (start 166.899214 38.705786) (end 164.715 40.89) (width 0.2) (layer "F.Cu") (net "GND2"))
 (segment (start 124.46 67.31) (end 124.46 54.61) (width 0.2) (layer "F.Cu") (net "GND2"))
 (segment (start 124.46 54.61) (end 132.08 46.99) (width 0.2) (layer "F.Cu") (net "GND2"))
 (segment (start 164.715 40.89) (end 139.315 40.89) (width 0.2) (layer "B.Cu") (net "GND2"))
 (segment (start 170.15 52.12) (end 151.08 52.12) (width 0.2) (layer "B.Cu") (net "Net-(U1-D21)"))
 (segment (start 140.054 62.23) (end 138.784 63.5) (width 0.2) (layer "B.Cu") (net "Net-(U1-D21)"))
 (segment (start 151.08 52.12) (end 140.97 62.23) (width 0.2) (layer "B.Cu") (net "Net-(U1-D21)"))
 (segment (start 140.97 62.23) (end 140.054 62.23) (width 0.2) (layer "B.Cu") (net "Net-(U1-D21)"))
 (segment (start 170.15 54.66) (end 155.244 54.66) (width 0.2) (layer "B.Cu") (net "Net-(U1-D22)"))
 (segment (start 155.244 54.66) (end 138.784 71.12) (width 0.2) (layer "B.Cu") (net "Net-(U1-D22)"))
 (segment (start 158.75 121.92) (end 154.94 118.11) (width 0.2) (layer "F.Cu") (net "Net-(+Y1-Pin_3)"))
 (segment (start 154.94 63.365) (end 164.715 53.59) (width 0.2) (layer "F.Cu") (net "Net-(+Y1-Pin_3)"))
 (segment (start 154.94 118.11) (end 154.94 63.365) (width 0.2) (layer "F.Cu") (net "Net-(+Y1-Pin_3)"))
 (segment (start 141.605 49.53) (end 141.605 58.139) (width 0.2) (layer "B.Cu") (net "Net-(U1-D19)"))
 (segment (start 132.08 49.53) (end 141.605 49.53) (width 0.2) (layer "B.Cu") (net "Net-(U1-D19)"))
 (segment (start 141.605 58.139) (end 138.784 60.96) (width 0.2) (layer "B.Cu") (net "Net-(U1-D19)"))
 (segment (start 138.43 58.42) (end 138.784 58.42) (width 0.2) (layer "B.Cu") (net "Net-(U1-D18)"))
 (segment (start 132.08 52.07) (end 138.43 58.42) (width 0.2) (layer "B.Cu") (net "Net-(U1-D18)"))
 (segment (start 129.54 64.416) (end 138.784 73.66) (width 0.2) (layer "B.Cu") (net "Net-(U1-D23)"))
 (segment (start 129.54 57.15) (end 129.54 64.416) (width 0.2) (layer "B.Cu") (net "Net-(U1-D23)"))
 (segment (start 132.08 54.61) (end 129.54 57.15) (width 0.2) (layer "B.Cu") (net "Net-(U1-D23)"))
 (segment (start 132.08 57.15) (end 133.35 55.88) (width 0.2) (layer "F.Cu") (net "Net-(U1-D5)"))
 (segment (start 133.35 55.88) (end 138.784 55.88) (width 0.2) (layer "F.Cu") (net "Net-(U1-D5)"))
 (segment (start 163.83 121.92) (end 157.48 115.57) (width 0.2) (layer "F.Cu") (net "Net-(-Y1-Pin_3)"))
 (segment (start 157.48 63.365) (end 164.715 56.13) (width 0.2) (layer "F.Cu") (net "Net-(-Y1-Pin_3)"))
 (segment (start 157.48 115.57) (end 157.48 63.365) (width 0.2) (layer "F.Cu") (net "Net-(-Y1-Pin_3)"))
 (segment (start 130.81 36.83) (end 130.81 33.02) (width 0.2) (layer "F.Cu") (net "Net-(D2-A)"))
 (segment (start 169.225 42.23) (end 139.734 42.23) (width 0.2) (layer "B.Cu") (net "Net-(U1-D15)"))
 (segment (start 170.18 41.275) (end 169.225 42.23) (width 0.2) (layer "B.Cu") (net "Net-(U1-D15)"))
 (segment (start 139.734 42.23) (end 138.784 43.18) (width 0.2) (layer "B.Cu") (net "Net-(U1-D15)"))
 (segment (start 134.62 45.72) (end 138.784 45.72) (width 0.2) (layer "B.Cu") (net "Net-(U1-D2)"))
 (segment (start 130.81 41.91) (end 134.62 45.72) (width 0.2) (layer "B.Cu") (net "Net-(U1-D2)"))
 (segment (start 144.78 115.57) (end 144.78 63.365) (width 0.2) (layer "F.Cu") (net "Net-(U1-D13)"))
 (segment (start 138.43 121.92) (end 144.78 115.57) (width 0.2) (layer "F.Cu") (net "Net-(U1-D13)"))
 (segment (start 144.78 63.365) (end 164.715 43.43) (width 0.2) (layer "F.Cu") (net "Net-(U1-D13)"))
 (segment (start 147.32 63.365) (end 164.715 45.97) (width 0.2) (layer "F.Cu") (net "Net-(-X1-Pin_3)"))
 (segment (start 143.51 121.92) (end 147.32 118.11) (width 0.2) (layer "F.Cu") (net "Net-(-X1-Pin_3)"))
 (segment (start 147.32 118.11) (end 147.32 63.365) (width 0.2) (layer "F.Cu") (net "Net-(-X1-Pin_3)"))
 (segment (start 149.86 63.365) (end 164.715 48.51) (width 0.2) (layer "F.Cu") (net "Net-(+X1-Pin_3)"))
 (segment (start 149.86 120.65) (end 149.86 63.365) (width 0.2) (layer "F.Cu") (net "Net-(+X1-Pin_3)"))
 (segment (start 148.59 121.92) (end 149.86 120.65) (width 0.2) (layer "F.Cu") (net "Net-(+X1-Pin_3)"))
 (segment (start 163.58 63.75) (end 164.715 63.75) (width 0.2) (layer "B.Cu") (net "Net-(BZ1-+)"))
 (segment (start 152.42 74.91) (end 163.58 63.75) (width 0.2) (layer "B.Cu") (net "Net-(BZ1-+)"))
 (segment (start 124.46 74.91) (end 152.42 74.91) (width 0.2) (layer "B.Cu") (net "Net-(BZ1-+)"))
 (segment (start 170.18 36.195) (end 170.18 33.02) (width 0.2) (layer "F.Cu") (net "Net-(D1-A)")))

